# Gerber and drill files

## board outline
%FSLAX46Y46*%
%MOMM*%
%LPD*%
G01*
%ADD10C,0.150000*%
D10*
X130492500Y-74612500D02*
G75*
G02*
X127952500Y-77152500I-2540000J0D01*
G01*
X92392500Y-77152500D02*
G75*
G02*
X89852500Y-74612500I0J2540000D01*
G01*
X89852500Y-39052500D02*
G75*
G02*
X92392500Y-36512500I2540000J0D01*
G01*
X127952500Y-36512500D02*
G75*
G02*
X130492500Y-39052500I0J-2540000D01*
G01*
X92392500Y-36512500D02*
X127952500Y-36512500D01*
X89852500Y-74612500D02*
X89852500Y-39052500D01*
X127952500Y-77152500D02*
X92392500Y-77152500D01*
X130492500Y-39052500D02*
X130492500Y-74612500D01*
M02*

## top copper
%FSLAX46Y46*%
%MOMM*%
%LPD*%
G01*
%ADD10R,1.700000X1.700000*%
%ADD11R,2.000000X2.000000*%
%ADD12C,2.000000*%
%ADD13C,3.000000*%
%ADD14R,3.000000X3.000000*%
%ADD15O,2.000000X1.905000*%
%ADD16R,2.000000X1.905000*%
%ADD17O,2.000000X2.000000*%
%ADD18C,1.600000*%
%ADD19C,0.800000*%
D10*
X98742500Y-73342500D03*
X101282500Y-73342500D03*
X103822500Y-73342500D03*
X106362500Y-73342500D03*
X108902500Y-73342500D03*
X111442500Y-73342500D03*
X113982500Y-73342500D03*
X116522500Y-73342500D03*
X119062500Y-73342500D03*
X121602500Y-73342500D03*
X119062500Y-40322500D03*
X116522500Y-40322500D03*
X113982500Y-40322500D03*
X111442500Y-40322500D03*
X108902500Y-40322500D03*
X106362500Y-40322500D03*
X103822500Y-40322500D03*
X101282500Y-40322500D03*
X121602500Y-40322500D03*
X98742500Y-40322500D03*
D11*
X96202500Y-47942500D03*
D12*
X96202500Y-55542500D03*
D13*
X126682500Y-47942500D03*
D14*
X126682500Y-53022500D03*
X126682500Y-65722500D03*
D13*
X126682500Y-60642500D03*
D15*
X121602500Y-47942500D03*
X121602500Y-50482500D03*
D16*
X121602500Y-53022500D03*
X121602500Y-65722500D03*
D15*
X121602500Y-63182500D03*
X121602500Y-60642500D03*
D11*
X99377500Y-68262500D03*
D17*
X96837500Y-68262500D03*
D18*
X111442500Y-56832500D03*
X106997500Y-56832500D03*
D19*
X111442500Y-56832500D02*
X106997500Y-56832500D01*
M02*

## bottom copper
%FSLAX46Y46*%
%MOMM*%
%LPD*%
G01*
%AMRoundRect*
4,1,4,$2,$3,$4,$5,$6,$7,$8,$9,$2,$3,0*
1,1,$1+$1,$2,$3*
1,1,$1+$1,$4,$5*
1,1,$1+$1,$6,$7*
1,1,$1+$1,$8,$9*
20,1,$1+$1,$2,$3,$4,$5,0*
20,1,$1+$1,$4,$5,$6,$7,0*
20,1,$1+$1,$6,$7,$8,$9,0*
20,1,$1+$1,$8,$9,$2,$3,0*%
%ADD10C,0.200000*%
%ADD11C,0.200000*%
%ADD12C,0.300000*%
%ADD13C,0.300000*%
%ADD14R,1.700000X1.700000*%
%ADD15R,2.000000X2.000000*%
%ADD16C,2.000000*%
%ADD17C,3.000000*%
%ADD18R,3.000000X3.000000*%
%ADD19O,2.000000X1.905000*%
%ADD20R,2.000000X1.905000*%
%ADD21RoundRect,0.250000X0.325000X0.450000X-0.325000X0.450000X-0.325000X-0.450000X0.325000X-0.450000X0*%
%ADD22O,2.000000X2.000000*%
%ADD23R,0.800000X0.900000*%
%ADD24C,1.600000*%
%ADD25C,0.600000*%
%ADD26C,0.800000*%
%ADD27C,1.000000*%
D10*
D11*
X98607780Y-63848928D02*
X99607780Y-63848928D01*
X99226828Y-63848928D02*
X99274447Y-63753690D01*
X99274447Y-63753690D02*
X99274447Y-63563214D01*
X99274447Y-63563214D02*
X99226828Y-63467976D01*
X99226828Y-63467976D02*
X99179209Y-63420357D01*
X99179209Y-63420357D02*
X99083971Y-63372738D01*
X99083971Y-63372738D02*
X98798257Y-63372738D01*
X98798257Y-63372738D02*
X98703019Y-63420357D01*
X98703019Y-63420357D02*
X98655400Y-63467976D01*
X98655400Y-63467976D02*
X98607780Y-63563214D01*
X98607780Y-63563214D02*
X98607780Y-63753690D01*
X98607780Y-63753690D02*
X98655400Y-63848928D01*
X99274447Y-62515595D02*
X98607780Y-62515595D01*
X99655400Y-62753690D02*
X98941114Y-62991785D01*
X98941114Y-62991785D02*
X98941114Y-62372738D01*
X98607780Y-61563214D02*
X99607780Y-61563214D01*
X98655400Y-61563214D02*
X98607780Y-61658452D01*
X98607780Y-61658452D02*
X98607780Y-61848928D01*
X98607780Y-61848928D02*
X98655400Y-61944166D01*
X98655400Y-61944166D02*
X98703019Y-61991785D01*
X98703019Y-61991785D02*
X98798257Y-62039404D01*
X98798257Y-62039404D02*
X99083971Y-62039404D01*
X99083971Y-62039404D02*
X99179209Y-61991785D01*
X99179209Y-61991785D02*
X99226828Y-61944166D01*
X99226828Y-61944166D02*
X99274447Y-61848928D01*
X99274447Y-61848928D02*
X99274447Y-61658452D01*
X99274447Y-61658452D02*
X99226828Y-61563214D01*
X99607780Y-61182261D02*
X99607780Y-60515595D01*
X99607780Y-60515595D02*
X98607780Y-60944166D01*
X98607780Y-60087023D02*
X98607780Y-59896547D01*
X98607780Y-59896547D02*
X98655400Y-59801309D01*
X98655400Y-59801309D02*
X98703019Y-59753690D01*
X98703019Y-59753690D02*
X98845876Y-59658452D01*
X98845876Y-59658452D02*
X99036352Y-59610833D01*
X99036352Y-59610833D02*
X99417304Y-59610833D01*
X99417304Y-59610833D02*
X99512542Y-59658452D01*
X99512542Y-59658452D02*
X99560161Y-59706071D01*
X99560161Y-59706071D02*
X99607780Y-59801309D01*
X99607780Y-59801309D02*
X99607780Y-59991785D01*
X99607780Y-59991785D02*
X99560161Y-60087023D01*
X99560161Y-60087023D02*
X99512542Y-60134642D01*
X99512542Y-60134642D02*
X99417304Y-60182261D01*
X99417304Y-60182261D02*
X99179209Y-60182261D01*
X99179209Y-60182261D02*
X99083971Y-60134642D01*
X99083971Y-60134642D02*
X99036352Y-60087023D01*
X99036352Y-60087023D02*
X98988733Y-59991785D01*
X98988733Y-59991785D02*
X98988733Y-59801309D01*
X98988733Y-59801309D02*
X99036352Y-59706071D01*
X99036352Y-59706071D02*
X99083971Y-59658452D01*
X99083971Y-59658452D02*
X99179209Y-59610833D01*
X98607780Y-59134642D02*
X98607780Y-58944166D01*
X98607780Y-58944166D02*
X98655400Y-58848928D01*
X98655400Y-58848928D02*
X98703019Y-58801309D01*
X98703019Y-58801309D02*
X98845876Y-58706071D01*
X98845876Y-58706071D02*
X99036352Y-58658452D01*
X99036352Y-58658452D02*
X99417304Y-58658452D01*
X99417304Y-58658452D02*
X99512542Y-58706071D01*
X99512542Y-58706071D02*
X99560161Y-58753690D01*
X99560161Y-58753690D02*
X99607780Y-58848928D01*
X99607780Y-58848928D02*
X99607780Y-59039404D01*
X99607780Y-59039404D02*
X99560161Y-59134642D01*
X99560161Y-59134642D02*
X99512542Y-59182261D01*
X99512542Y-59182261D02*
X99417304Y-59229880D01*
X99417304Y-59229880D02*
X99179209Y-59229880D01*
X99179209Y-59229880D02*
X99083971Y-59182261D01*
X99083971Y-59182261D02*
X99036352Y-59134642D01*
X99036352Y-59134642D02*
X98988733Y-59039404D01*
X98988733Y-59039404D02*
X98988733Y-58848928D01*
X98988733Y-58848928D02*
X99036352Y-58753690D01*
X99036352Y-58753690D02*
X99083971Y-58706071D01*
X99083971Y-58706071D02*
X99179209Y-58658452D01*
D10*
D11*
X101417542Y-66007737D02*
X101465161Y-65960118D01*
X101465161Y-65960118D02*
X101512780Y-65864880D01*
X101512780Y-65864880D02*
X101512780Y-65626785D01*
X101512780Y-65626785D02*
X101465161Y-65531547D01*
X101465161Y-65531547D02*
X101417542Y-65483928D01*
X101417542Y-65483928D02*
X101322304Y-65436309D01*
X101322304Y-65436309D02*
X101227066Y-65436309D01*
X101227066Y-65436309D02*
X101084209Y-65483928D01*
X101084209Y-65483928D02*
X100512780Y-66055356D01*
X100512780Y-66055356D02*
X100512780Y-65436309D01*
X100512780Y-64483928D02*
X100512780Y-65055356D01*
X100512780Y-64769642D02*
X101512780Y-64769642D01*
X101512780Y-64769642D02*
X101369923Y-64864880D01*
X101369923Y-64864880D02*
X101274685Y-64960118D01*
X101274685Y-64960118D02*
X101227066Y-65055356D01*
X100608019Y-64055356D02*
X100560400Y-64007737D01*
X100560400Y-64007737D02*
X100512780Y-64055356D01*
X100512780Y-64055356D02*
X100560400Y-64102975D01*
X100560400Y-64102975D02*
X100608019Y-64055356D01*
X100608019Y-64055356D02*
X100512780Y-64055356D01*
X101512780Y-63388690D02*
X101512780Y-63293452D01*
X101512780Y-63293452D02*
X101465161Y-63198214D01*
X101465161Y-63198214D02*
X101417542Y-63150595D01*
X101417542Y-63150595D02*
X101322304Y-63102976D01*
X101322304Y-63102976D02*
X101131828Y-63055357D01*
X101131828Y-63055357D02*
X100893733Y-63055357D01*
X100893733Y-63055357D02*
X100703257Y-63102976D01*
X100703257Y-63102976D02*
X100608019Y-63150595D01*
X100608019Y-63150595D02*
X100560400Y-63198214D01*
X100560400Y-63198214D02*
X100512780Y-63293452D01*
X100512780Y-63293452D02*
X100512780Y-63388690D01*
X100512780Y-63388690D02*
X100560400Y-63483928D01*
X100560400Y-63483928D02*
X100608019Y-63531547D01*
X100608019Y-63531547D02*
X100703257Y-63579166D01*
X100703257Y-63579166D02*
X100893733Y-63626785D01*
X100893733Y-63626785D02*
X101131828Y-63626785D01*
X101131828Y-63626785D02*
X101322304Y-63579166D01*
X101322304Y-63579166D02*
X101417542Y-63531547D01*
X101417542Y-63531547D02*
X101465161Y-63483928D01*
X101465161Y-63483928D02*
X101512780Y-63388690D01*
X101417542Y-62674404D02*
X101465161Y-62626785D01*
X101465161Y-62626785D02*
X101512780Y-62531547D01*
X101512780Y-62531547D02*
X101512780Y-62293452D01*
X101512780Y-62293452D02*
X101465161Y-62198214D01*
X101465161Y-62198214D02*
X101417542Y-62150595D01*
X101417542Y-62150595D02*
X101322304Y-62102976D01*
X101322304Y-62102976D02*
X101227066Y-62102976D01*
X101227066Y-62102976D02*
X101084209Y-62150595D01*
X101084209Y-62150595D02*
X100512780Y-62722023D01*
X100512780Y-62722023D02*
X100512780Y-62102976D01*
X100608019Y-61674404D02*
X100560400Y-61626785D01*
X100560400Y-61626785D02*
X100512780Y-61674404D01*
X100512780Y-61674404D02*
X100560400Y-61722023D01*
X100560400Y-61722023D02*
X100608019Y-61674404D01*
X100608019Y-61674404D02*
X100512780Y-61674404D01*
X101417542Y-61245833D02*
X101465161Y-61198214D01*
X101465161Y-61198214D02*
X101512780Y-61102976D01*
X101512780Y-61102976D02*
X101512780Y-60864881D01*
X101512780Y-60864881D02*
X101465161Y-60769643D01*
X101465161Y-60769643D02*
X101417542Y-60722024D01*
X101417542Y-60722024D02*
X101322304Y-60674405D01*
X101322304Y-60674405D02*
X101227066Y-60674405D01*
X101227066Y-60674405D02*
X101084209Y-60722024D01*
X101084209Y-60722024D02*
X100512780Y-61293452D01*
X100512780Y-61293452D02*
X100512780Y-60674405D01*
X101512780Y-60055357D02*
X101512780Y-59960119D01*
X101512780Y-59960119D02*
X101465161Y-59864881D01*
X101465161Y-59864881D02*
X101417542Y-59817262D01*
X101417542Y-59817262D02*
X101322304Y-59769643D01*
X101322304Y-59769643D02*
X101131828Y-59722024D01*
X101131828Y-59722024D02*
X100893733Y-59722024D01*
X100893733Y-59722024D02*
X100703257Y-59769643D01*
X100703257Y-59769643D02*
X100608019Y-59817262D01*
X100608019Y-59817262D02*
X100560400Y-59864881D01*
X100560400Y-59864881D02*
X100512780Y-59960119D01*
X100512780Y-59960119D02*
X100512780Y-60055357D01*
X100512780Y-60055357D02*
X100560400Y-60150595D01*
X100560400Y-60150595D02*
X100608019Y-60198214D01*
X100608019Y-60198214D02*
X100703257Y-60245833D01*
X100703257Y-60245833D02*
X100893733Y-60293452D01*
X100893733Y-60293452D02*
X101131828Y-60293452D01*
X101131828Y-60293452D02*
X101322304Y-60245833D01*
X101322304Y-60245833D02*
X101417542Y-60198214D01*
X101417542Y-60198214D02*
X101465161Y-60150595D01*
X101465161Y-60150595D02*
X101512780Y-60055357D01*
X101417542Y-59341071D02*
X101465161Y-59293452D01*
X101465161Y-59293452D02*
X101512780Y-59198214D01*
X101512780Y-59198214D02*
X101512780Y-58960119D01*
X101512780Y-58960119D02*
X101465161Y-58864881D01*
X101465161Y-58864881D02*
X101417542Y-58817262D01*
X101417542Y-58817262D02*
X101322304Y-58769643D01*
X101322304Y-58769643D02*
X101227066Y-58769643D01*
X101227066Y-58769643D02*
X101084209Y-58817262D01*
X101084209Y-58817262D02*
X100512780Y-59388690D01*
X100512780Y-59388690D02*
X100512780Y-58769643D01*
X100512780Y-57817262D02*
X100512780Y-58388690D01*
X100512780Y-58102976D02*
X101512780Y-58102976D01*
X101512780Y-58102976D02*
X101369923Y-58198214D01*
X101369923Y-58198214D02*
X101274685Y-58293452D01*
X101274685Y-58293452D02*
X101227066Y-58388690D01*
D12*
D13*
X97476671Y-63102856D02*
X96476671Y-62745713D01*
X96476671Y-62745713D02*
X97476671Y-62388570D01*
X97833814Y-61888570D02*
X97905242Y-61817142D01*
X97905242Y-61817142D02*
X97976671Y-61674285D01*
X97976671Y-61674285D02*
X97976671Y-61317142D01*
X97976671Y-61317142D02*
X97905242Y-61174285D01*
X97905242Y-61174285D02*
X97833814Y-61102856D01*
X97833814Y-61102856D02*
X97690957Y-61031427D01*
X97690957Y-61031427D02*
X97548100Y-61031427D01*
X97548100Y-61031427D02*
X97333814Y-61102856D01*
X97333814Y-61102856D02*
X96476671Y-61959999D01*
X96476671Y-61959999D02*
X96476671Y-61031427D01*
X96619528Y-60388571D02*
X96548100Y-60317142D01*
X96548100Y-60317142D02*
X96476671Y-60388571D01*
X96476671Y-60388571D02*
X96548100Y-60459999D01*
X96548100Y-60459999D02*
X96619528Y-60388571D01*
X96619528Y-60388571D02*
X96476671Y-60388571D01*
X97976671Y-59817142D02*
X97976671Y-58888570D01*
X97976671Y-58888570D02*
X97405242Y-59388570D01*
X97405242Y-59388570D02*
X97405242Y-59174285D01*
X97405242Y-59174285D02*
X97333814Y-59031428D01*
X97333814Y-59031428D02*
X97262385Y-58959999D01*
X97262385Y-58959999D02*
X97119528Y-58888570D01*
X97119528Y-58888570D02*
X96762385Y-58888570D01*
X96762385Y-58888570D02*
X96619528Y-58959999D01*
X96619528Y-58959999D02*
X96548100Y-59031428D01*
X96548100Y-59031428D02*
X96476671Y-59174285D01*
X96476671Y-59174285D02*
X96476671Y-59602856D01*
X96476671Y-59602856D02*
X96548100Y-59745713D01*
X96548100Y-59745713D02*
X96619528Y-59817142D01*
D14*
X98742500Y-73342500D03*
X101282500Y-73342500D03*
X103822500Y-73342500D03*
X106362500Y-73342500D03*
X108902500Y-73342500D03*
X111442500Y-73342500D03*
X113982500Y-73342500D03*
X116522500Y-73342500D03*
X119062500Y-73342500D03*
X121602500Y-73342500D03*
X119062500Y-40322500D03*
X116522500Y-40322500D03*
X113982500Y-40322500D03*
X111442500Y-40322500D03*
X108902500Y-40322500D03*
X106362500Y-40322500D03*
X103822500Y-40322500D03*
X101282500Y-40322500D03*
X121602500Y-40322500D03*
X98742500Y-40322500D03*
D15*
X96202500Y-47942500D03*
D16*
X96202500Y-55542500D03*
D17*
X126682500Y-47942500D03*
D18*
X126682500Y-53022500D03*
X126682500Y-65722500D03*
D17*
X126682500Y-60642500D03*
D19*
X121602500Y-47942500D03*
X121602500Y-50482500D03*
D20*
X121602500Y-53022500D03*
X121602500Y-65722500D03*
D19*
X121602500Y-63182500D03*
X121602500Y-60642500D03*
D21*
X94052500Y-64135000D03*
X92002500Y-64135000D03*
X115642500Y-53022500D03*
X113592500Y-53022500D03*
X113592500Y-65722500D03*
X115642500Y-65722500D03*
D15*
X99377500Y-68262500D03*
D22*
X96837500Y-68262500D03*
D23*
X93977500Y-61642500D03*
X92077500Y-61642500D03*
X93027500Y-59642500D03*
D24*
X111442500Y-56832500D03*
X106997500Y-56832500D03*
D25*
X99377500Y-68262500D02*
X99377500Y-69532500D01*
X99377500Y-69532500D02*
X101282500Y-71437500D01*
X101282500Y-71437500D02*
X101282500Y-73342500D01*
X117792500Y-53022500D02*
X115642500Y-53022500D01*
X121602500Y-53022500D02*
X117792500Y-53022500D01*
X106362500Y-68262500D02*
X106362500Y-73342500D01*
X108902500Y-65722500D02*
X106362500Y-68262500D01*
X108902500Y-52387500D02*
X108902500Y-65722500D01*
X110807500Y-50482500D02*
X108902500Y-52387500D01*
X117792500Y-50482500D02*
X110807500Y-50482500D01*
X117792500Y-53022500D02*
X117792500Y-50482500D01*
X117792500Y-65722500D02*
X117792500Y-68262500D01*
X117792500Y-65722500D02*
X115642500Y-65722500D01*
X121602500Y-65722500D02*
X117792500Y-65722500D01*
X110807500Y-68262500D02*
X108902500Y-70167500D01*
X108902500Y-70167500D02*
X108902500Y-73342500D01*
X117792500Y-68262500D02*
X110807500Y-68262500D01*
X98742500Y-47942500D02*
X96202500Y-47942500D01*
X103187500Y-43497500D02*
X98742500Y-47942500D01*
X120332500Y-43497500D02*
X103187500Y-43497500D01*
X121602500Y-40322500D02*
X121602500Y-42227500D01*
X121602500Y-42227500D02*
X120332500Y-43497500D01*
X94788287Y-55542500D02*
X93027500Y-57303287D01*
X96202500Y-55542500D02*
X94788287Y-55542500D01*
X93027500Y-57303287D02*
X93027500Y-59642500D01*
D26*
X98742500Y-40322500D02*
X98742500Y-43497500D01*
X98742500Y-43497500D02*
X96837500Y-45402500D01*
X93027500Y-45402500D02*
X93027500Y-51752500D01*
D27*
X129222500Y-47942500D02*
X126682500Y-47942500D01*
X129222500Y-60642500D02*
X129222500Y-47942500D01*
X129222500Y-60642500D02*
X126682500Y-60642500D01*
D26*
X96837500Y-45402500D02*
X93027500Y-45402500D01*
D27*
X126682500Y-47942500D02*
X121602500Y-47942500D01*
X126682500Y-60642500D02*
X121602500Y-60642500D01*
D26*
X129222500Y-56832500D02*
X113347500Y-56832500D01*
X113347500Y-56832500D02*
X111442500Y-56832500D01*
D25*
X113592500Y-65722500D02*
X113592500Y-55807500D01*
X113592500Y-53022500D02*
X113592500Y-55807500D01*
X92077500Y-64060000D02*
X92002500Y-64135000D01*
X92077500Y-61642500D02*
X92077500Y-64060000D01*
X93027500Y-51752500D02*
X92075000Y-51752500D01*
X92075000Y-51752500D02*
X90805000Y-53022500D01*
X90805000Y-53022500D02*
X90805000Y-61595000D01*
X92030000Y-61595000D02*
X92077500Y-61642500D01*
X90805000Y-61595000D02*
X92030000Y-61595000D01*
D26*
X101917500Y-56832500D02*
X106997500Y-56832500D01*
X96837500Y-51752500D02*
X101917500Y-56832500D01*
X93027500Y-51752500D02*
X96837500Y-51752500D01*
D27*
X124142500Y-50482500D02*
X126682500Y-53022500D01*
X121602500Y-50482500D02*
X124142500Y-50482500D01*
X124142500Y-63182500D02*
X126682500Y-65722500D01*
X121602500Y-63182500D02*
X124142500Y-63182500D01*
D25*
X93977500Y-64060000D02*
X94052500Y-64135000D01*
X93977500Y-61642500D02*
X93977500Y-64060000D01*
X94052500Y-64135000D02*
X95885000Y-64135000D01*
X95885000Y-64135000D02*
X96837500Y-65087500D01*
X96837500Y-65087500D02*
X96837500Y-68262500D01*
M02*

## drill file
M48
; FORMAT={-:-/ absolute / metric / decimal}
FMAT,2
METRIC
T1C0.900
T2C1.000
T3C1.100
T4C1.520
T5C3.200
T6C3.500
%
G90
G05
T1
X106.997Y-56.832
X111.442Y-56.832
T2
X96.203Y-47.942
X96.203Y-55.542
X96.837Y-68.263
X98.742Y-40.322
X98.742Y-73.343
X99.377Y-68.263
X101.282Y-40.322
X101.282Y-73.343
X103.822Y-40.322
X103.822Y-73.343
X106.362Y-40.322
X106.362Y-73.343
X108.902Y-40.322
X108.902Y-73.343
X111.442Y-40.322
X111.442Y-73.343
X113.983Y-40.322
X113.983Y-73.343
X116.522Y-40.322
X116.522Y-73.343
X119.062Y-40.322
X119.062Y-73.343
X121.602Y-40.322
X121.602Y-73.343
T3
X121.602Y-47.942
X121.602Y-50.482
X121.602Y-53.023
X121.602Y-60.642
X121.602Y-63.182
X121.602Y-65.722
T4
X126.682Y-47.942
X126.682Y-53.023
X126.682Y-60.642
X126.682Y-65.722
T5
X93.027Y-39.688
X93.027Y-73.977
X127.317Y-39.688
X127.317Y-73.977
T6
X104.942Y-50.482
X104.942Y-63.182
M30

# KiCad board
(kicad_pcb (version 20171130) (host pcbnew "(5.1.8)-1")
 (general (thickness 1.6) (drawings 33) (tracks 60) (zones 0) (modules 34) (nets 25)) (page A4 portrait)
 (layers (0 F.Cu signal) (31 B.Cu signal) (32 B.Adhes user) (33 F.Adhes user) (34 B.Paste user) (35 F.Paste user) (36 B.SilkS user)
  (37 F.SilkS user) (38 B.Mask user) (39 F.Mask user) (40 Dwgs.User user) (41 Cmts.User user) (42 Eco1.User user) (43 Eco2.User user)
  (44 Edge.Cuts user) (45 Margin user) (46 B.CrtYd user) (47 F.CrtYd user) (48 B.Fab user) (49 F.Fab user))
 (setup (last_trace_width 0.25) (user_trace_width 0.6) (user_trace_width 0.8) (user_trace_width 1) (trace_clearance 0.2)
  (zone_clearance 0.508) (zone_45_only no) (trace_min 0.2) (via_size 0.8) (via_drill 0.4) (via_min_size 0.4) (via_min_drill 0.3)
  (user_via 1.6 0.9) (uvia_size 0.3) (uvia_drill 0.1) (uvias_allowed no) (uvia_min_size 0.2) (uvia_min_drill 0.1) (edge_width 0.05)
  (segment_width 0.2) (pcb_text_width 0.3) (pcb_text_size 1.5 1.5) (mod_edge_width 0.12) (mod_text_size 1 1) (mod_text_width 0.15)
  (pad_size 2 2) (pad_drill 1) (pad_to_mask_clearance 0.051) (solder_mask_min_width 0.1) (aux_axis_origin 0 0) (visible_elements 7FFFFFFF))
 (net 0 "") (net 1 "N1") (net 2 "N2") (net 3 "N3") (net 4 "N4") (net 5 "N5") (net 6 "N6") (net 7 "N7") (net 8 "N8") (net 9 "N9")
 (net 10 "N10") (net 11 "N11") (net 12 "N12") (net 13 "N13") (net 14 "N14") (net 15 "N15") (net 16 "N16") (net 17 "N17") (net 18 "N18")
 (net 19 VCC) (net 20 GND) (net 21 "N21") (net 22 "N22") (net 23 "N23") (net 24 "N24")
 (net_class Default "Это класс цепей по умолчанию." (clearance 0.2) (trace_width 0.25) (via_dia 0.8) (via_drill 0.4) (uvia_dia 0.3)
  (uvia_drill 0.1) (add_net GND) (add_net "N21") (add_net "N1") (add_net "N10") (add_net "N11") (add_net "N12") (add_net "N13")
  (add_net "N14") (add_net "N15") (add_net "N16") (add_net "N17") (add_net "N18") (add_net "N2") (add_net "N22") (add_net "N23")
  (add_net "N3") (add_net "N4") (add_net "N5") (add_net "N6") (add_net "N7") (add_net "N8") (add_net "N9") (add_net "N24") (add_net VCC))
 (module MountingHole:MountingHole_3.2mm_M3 (layer F.Cu) (at 127.3175 39.6875 270)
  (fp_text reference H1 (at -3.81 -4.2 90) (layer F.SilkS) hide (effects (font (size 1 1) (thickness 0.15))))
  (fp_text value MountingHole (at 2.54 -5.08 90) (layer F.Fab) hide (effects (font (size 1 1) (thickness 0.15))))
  (pad 1 np_thru_hole circle (at 0 0 270) (size 3.2 3.2) (drill 3.2) (layers *.Cu *.Mask)))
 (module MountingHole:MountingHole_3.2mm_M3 (layer F.Cu) (at 93.0275 39.6875 270)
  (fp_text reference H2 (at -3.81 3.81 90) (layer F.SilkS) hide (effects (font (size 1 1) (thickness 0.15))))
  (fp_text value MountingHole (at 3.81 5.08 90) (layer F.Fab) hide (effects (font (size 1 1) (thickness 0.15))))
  (pad 1 np_thru_hole circle (at 0 0 270) (size 3.2 3.2) (drill 3.2) (layers *.Cu *.Mask)))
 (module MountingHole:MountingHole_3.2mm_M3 (layer F.Cu) (at 127.3175 73.9775 270)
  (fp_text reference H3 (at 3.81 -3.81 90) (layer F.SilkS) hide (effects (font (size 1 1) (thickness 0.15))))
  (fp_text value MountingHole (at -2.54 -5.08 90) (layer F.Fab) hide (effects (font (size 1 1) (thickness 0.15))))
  (pad 1 np_thru_hole circle (at 0 0 270) (size 3.2 3.2) (drill 3.2) (layers *.Cu *.Mask)))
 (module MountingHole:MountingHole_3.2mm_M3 (layer F.Cu) (at 93.0275 73.9775 270)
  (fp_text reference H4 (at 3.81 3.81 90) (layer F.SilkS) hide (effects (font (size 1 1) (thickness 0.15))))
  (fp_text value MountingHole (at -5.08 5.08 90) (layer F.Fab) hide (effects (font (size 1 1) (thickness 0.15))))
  (pad 1 np_thru_hole circle (at 0 0 270) (size 3.2 3.2) (drill 3.2) (layers *.Cu *.Mask)))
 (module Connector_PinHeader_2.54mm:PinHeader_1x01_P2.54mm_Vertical (layer F.Cu) (at 98.7425 73.3425 270)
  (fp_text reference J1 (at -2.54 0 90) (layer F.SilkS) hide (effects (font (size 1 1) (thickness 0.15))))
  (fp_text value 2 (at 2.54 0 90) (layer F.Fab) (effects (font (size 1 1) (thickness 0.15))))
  (pad 1 thru_hole rect (at 0 0 270) (size 1.7 1.7) (drill 1) (layers *.Cu *.Mask) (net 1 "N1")))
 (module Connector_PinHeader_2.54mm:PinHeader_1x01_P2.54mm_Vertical (layer F.Cu) (at 101.2825 73.3425 270)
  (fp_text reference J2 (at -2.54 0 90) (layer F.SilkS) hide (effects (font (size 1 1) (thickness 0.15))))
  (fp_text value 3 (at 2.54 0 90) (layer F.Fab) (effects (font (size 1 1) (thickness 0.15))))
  (pad 1 thru_hole rect (at 0 0 270) (size 1.7 1.7) (drill 1) (layers *.Cu *.Mask) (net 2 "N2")))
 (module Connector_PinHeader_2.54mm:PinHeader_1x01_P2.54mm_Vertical (layer F.Cu) (at 103.8225 73.3425 270)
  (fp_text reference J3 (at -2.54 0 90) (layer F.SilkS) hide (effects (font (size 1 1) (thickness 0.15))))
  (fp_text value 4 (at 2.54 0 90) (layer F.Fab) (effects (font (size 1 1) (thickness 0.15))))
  (pad 1 thru_hole rect (at 0 0 270) (size 1.7 1.7) (drill 1) (layers *.Cu *.Mask) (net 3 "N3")))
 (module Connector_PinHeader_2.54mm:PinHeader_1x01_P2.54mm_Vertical (layer F.Cu) (at 106.3625 73.3425 270)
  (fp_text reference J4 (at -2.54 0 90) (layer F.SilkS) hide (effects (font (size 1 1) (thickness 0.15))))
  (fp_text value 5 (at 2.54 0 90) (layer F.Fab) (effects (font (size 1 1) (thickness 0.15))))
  (pad 1 thru_hole rect (at 0 0 270) (size 1.7 1.7) (drill 1) (layers *.Cu *.Mask) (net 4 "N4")))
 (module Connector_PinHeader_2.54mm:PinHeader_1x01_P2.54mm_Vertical (layer F.Cu) (at 108.9025 73.3425 270)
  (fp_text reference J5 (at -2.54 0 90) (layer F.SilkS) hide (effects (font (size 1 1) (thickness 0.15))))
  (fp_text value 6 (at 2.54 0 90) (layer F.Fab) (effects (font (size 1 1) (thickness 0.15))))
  (pad 1 thru_hole rect (at 0 0 270) (size 1.7 1.7) (drill 1) (layers *.Cu *.Mask) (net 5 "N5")))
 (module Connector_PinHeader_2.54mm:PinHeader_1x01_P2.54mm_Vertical (layer F.Cu) (at 111.4425 73.3425 270)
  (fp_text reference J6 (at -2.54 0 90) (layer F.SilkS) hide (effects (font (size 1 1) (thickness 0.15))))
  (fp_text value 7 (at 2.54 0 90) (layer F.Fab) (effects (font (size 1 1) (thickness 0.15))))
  (pad 1 thru_hole rect (at 0 0 270) (size 1.7 1.7) (drill 1) (layers *.Cu *.Mask) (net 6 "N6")))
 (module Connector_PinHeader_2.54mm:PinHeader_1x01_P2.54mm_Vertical (layer F.Cu) (at 113.9825 73.3425 270)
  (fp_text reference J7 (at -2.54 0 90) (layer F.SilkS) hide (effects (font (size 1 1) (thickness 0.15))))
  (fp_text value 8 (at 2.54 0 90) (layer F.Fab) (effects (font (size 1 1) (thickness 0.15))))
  (pad 1 thru_hole rect (at 0 0 270) (size 1.7 1.7) (drill 1) (layers *.Cu *.Mask) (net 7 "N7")))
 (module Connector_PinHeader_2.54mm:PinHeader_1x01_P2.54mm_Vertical (layer F.Cu) (at 116.5225 73.3425 270)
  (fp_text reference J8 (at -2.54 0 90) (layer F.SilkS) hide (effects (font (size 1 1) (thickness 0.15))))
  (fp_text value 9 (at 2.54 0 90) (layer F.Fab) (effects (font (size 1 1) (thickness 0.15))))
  (pad 1 thru_hole rect (at 0 0 270) (size 1.7 1.7) (drill 1) (layers *.Cu *.Mask) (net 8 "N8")))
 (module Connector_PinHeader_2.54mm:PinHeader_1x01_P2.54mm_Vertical (layer F.Cu) (at 119.0625 73.3425 270)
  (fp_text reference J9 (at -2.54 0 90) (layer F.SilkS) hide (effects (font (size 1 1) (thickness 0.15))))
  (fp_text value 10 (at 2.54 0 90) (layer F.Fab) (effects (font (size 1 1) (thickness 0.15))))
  (pad 1 thru_hole rect (at 0 0 270) (size 1.7 1.7) (drill 1) (layers *.Cu *.Mask) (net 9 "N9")))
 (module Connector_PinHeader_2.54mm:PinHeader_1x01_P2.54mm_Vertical (layer F.Cu) (at 121.6025 73.3425 270)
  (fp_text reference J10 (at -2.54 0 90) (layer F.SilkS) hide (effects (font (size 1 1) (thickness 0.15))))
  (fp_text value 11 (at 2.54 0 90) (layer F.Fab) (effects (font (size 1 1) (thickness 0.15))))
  (pad 1 thru_hole rect (at 0 0 270) (size 1.7 1.7) (drill 1) (layers *.Cu *.Mask) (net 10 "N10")))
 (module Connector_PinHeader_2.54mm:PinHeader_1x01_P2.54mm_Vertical (layer F.Cu) (at 119.0625 40.3225 270)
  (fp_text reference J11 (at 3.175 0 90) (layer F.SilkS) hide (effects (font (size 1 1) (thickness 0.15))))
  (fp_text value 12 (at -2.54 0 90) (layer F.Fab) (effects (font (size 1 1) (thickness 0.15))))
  (pad 1 thru_hole rect (at 0 0 270) (size 1.7 1.7) (drill 1) (layers *.Cu *.Mask) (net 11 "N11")))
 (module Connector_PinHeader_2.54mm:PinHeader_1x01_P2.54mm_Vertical (layer F.Cu) (at 116.5225 40.3225 270)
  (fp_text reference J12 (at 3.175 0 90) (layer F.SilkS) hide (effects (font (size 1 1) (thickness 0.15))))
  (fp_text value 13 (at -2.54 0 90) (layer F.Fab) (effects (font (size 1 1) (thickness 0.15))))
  (pad 1 thru_hole rect (at 0 0 270) (size 1.7 1.7) (drill 1) (layers *.Cu *.Mask) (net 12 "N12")))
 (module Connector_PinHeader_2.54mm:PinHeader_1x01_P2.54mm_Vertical (layer F.Cu) (at 113.9825 40.3225 270)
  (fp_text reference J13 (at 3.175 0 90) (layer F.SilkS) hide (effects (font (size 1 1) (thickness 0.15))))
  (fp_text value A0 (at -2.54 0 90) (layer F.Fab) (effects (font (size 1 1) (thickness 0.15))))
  (pad 1 thru_hole rect (at 0 0 270) (size 1.7 1.7) (drill 1) (layers *.Cu *.Mask) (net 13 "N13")))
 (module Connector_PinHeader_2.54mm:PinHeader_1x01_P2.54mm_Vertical (layer F.Cu) (at 111.4425 40.3225 270)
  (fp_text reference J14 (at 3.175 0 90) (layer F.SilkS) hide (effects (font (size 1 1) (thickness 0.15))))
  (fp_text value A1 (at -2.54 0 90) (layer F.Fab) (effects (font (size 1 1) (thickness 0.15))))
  (pad 1 thru_hole rect (at 0 0 270) (size 1.7 1.7) (drill 1) (layers *.Cu *.Mask) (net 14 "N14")))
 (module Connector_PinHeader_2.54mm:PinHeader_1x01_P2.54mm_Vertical (layer F.Cu) (at 108.9025 40.3225 270)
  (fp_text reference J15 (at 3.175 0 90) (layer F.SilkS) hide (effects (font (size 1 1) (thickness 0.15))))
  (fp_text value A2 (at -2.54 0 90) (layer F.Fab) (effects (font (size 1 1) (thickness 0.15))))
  (pad 1 thru_hole rect (at 0 0 270) (size 1.7 1.7) (drill 1) (layers *.Cu *.Mask) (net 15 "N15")))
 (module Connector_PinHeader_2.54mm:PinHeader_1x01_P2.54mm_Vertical (layer F.Cu) (at 106.3625 40.3225 270)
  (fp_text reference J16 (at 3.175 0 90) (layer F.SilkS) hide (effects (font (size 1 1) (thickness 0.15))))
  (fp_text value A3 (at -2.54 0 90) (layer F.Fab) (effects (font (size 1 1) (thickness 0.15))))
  (pad 1 thru_hole rect (at 0 0 270) (size 1.7 1.7) (drill 1) (layers *.Cu *.Mask) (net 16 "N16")))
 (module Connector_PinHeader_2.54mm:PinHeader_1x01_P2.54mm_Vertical (layer F.Cu) (at 103.8225 40.3225 270)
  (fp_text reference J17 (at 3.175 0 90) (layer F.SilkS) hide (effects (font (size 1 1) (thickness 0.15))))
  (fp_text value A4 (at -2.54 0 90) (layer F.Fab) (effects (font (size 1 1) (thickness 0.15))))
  (pad 1 thru_hole rect (at 0 0 270) (size 1.7 1.7) (drill 1) (layers *.Cu *.Mask) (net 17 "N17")))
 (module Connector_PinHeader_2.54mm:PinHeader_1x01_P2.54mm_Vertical (layer F.Cu) (at 101.2825 40.3225 270)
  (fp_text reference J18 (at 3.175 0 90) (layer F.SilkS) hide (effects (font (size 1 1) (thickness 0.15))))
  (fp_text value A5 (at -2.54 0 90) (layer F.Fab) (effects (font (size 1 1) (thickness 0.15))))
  (pad 1 thru_hole rect (at 0 0 270) (size 1.7 1.7) (drill 1) (layers *.Cu *.Mask) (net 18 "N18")))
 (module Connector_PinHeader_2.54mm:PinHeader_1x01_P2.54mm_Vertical (layer F.Cu) (at 121.6025 40.3225 270)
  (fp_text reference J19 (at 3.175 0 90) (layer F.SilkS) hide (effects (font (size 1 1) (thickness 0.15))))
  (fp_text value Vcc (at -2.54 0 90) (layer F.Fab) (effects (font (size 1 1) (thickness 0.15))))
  (pad 1 thru_hole rect (at 0 0 270) (size 1.7 1.7) (drill 1) (layers *.Cu *.Mask) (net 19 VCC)))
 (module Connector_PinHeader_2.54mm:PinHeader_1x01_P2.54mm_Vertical (layer F.Cu) (at 98.7425 40.3225 270)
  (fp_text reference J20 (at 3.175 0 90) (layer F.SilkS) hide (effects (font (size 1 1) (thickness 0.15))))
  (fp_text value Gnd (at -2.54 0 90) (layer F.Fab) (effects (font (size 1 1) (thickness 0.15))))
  (pad 1 thru_hole rect (at 0 0 270) (size 1.7 1.7) (drill 1) (layers *.Cu *.Mask) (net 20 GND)))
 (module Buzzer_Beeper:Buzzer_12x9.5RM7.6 (layer F.Cu) (at 96.2025 47.9425 270)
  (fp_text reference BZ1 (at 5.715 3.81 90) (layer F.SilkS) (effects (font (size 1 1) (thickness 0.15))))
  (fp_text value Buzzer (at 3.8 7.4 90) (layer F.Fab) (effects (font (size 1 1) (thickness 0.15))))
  (pad 1 thru_hole rect (at 0 0 270) (size 2 2) (drill 1) (layers *.Cu *.Mask) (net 19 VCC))
  (pad 2 thru_hole circle (at 7.6 0 270) (size 2 2) (drill 1) (layers *.Cu *.Mask) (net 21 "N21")))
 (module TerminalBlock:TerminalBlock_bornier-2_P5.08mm (layer F.Cu) (at 126.6825 53.0225 90)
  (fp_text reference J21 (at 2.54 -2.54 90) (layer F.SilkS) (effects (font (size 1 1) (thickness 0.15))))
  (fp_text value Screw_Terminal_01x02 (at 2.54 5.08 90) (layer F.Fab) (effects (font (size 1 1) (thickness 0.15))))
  (pad 2 thru_hole circle (at 5.08 0 90) (size 3 3) (drill 1.52) (layers *.Cu *.Mask) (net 20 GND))
  (pad 1 thru_hole rect (at 0 0 90) (size 3 3) (drill 1.52) (layers *.Cu *.Mask) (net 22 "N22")))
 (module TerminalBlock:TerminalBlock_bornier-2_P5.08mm (layer F.Cu) (at 126.6825 65.7225 90)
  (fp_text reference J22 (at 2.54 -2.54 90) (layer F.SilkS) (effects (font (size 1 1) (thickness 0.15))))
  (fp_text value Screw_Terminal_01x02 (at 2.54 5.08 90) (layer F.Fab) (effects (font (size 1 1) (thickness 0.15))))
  (pad 1 thru_hole rect (at 0 0 90) (size 3 3) (drill 1.52) (layers *.Cu *.Mask) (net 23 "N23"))
  (pad 2 thru_hole circle (at 5.08 0 90) (size 3 3) (drill 1.52) (layers *.Cu *.Mask) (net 20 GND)))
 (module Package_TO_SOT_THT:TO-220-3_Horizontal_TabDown (layer F.Cu) (at 121.6025 53.0225 90)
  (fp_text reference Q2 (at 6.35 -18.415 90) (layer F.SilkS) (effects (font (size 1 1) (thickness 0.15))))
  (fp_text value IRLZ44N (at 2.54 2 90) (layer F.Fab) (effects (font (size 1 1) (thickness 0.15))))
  (pad 3 thru_hole oval (at 5.08 0 90) (size 1.905 2) (drill 1.1) (layers *.Cu *.Mask) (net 20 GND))
  (pad 2 thru_hole oval (at 2.54 0 90) (size 1.905 2) (drill 1.1) (layers *.Cu *.Mask) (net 22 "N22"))
  (pad 1 thru_hole rect (at 0 0 90) (size 1.905 2) (drill 1.1) (layers *.Cu *.Mask) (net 4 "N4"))
  (pad "" np_thru_hole oval (at 2.54 -16.66 90) (size 3.5 3.5) (drill 3.5) (layers *.Cu *.Mask)))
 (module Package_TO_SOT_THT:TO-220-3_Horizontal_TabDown (layer F.Cu) (at 121.6025 65.7225 90)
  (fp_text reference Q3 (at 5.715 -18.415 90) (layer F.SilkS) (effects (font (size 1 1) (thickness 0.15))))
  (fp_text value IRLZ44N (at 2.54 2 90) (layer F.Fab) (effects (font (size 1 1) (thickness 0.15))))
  (pad "" np_thru_hole oval (at 2.54 -16.66 90) (size 3.5 3.5) (drill 3.5) (layers *.Cu *.Mask))
  (pad 1 thru_hole rect (at 0 0 90) (size 1.905 2) (drill 1.1) (layers *.Cu *.Mask) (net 5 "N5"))
  (pad 2 thru_hole oval (at 2.54 0 90) (size 1.905 2) (drill 1.1) (layers *.Cu *.Mask) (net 23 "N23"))
  (pad 3 thru_hole oval (at 5.08 0 90) (size 1.905 2) (drill 1.1) (layers *.Cu *.Mask) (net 20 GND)))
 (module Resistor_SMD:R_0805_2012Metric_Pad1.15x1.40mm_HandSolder (layer B.Cu) (at 93.0275 64.135 180)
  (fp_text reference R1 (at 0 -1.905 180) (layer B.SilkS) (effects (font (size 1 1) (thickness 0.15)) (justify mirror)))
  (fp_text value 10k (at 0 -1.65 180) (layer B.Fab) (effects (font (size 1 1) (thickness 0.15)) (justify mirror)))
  (pad 1 smd roundrect (at -1.025 0 180) (size 1.15 1.4) (layers B.Cu B.Paste B.Mask) (roundrect_rratio 0.217391) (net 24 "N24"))
  (pad 2 smd roundrect (at 1.025 0 180) (size 1.15 1.4) (layers B.Cu B.Paste B.Mask) (roundrect_rratio 0.217391) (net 20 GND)))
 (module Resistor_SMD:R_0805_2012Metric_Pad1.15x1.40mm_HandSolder (layer B.Cu) (at 114.6175 53.0225 180)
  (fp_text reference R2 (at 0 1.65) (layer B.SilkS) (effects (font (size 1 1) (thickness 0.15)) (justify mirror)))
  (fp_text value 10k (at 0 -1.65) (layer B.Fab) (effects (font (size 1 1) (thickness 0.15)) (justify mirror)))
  (pad 1 smd roundrect (at -1.025 0 180) (size 1.15 1.4) (layers B.Cu B.Paste B.Mask) (roundrect_rratio 0.217391) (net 4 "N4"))
  (pad 2 smd roundrect (at 1.025 0 180) (size 1.15 1.4) (layers B.Cu B.Paste B.Mask) (roundrect_rratio 0.217391) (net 20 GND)))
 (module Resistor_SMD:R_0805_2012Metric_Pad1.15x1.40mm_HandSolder (layer B.Cu) (at 114.6175 65.7225 180)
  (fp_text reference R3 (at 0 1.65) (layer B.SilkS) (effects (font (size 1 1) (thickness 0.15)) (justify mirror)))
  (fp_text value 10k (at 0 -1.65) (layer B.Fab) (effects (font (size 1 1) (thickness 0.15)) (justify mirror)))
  (pad 2 smd roundrect (at 1.025 0 180) (size 1.15 1.4) (layers B.Cu B.Paste B.Mask) (roundrect_rratio 0.217391) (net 20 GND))
  (pad 1 smd roundrect (at -1.025 0 180) (size 1.15 1.4) (layers B.Cu B.Paste B.Mask) (roundrect_rratio 0.217391) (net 5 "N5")))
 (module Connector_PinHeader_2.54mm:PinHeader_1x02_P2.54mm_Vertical (layer F.Cu) (at 99.3775 68.2625 270)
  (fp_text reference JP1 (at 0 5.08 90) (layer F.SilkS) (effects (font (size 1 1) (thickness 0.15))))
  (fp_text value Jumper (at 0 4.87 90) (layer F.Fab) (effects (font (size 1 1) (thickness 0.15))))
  (pad 1 thru_hole rect (at 0 0 270) (size 2 2) (drill 1) (layers *.Cu *.Mask) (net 2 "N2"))
  (pad 2 thru_hole oval (at 0 2.54 270) (size 2 2) (drill 1) (layers *.Cu *.Mask) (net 24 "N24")))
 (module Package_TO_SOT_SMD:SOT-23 (layer B.Cu) (at 93.0275 60.6425 90)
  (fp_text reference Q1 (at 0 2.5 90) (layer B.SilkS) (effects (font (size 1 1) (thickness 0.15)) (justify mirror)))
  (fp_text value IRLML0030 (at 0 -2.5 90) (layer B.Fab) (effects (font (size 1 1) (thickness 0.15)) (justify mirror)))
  (pad 1 smd rect (at -1 0.95 90) (size 0.9 0.8) (layers B.Cu B.Paste B.Mask) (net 24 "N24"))
  (pad 2 smd rect (at -1 -0.95 90) (size 0.9 0.8) (layers B.Cu B.Paste B.Mask) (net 20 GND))
  (pad 3 smd rect (at 1 0 90) (size 0.9 0.8) (layers B.Cu B.Paste B.Mask) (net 21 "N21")))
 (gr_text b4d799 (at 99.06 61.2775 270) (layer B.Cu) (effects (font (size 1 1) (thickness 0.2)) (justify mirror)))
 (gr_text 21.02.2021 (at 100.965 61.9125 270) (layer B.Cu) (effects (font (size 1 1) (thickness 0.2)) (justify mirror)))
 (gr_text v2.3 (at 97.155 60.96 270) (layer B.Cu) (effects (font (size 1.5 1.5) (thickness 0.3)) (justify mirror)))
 (gr_arc (start 127.9525 74.6125) (end 127.9525 77.1525) (angle -90) (layer Edge.Cuts) (width 0.15))
 (gr_arc (start 92.3925 74.6125) (end 89.8525 74.6125) (angle -90) (layer Edge.Cuts) (width 0.15))
 (gr_arc (start 92.3925 39.0525) (end 92.3925 36.5125) (angle -90) (layer Edge.Cuts) (width 0.15))
 (gr_arc (start 127.9525 39.0525) (end 130.4925 39.0525) (angle -90) (layer Edge.Cuts) (width 0.15))
 (gr_line (start 92.3925 36.5125) (end 127.9525 36.5125) (layer Edge.Cuts) (width 0.15))
 (gr_line (start 89.8525 74.6125) (end 89.8525 39.0525) (layer Edge.Cuts) (width 0.15))
 (gr_line (start 127.9525 77.1525) (end 92.3925 77.1525) (layer Edge.Cuts) (width 0.15))
 (gr_line (start 130.4925 39.0525) (end 130.4925 74.6125) (layer Edge.Cuts) (width 0.15))
 (segment (start 99.3775 68.2625) (end 99.3775 69.5325) (width 0.6) (layer B.Cu) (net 2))
 (segment (start 99.3775 69.5325) (end 101.2825 71.4375) (width 0.6) (layer B.Cu) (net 2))
 (segment (start 101.2825 71.4375) (end 101.2825 73.3425) (width 0.6) (layer B.Cu) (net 2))
 (segment (start 117.7925 53.0225) (end 115.6425 53.0225) (width 0.6) (layer B.Cu) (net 4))
 (segment (start 121.6025 53.0225) (end 117.7925 53.0225) (width 0.6) (layer B.Cu) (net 4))
 (segment (start 106.3625 68.2625) (end 106.3625 73.3425) (width 0.6) (layer B.Cu) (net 4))
 (segment (start 108.9025 65.7225) (end 106.3625 68.2625) (width 0.6) (layer B.Cu) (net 4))
 (segment (start 108.9025 52.3875) (end 108.9025 65.7225) (width 0.6) (layer B.Cu) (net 4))
 (segment (start 110.8075 50.4825) (end 108.9025 52.3875) (width 0.6) (layer B.Cu) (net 4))
 (segment (start 117.7925 50.4825) (end 110.8075 50.4825) (width 0.6) (layer B.Cu) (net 4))
 (segment (start 117.7925 53.0225) (end 117.7925 50.4825) (width 0.6) (layer B.Cu) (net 4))
 (segment (start 117.7925 65.7225) (end 117.7925 68.2625) (width 0.6) (layer B.Cu) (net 5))
 (segment (start 117.7925 65.7225) (end 115.6425 65.7225) (width 0.6) (layer B.Cu) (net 5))
 (segment (start 121.6025 65.7225) (end 117.7925 65.7225) (width 0.6) (layer B.Cu) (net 5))
 (segment (start 110.8075 68.2625) (end 108.9025 70.1675) (width 0.6) (layer B.Cu) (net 5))
 (segment (start 108.9025 70.1675) (end 108.9025 73.3425) (width 0.6) (layer B.Cu) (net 5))
 (segment (start 117.7925 68.2625) (end 110.8075 68.2625) (width 0.6) (layer B.Cu) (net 5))
 (segment (start 98.7425 47.9425) (end 96.2025 47.9425) (width 0.6) (layer B.Cu) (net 19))
 (segment (start 103.1875 43.4975) (end 98.7425 47.9425) (width 0.6) (layer B.Cu) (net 19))
 (segment (start 120.3325 43.4975) (end 103.1875 43.4975) (width 0.6) (layer B.Cu) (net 19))
 (segment (start 121.6025 40.3225) (end 121.6025 42.2275) (width 0.6) (layer B.Cu) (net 19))
 (segment (start 121.6025 42.2275) (end 120.3325 43.4975) (width 0.6) (layer B.Cu) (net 19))
 (segment (start 94.788287 55.5425) (end 93.0275 57.303287) (width 0.6) (layer B.Cu) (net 21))
 (segment (start 96.2025 55.5425) (end 94.788287 55.5425) (width 0.6) (layer B.Cu) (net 21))
 (segment (start 93.0275 57.303287) (end 93.0275 59.6425) (width 0.6) (layer B.Cu) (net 21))
 (segment (start 98.7425 40.3225) (end 98.7425 43.4975) (width 0.8) (layer B.Cu) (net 20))
 (segment (start 98.7425 43.4975) (end 96.8375 45.4025) (width 0.8) (layer B.Cu) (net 20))
 (segment (start 93.0275 45.4025) (end 93.0275 51.7525) (width 0.8) (layer B.Cu) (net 20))
 (via (at 111.4425 56.8325) (size 1.6) (drill 0.9) (layers F.Cu B.Cu) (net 20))
 (via (at 106.9975 56.8325) (size 1.6) (drill 0.9) (layers F.Cu B.Cu) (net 20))
 (segment (start 111.4425 56.8325) (end 106.9975 56.8325) (width 0.8) (layer F.Cu) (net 20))
 (segment (start 129.2225 47.9425) (end 126.6825 47.9425) (width 1) (layer B.Cu) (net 20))
 (segment (start 129.2225 60.6425) (end 129.2225 47.9425) (width 1) (layer B.Cu) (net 20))
 (segment (start 129.2225 60.6425) (end 126.6825 60.6425) (width 1) (layer B.Cu) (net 20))
 (segment (start 96.8375 45.4025) (end 93.0275 45.4025) (width 0.8) (layer B.Cu) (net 20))
 (segment (start 126.6825 47.9425) (end 121.6025 47.9425) (width 1) (layer B.Cu) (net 20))
 (segment (start 126.6825 60.6425) (end 121.6025 60.6425) (width 1) (layer B.Cu) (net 20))
 (segment (start 129.2225 56.8325) (end 113.3475 56.8325) (width 0.8) (layer B.Cu) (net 20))
 (segment (start 113.3475 56.8325) (end 111.4425 56.8325) (width 0.8) (layer B.Cu) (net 20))
 (segment (start 113.5925 65.7225) (end 113.5925 55.8075) (width 0.6) (layer B.Cu) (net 20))
 (segment (start 113.5925 53.0225) (end 113.5925 55.8075) (width 0.6) (layer B.Cu) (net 20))
 (segment (start 92.0775 64.06) (end 92.0025 64.135) (width 0.6) (layer B.Cu) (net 20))
 (segment (start 92.0775 61.6425) (end 92.0775 64.06) (width 0.6) (layer B.Cu) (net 20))
 (segment (start 93.0275 51.7525) (end 92.075 51.7525) (width 0.6) (layer B.Cu) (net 20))
 (segment (start 92.075 51.7525) (end 90.805 53.0225) (width 0.6) (layer B.Cu) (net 20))
 (segment (start 90.805 53.0225) (end 90.805 61.595) (width 0.6) (layer B.Cu) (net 20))
 (segment (start 92.03 61.595) (end 92.0775 61.6425) (width 0.6) (layer B.Cu) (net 20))
 (segment (start 90.805 61.595) (end 92.03 61.595) (width 0.6) (layer B.Cu) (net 20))
 (segment (start 101.9175 56.8325) (end 106.9975 56.8325) (width 0.8) (layer B.Cu) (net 20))
 (segment (start 96.8375 51.7525) (end 101.9175 56.8325) (width 0.8) (layer B.Cu) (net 20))
 (segment (start 93.0275 51.7525) (end 96.8375 51.7525) (width 0.8) (layer B.Cu) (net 20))
 (segment (start 124.1425 50.4825) (end 126.6825 53.0225) (width 1) (layer B.Cu) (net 22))
 (segment (start 121.6025 50.4825) (end 124.1425 50.4825) (width 1) (layer B.Cu) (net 22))
 (segment (start 124.1425 63.1825) (end 126.6825 65.7225) (width 1) (layer B.Cu) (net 23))
 (segment (start 121.6025 63.1825) (end 124.1425 63.1825) (width 1) (layer B.Cu) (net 23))
 (segment (start 93.9775 64.06) (end 94.0525 64.135) (width 0.6) (layer B.Cu) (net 24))
 (segment (start 93.9775 61.6425) (end 93.9775 64.06) (width 0.6) (layer B.Cu) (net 24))
 (segment (start 94.0525 64.135) (end 95.885 64.135) (width 0.6) (layer B.Cu) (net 24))
 (segment (start 95.885 64.135) (end 96.8375 65.0875) (width 0.6) (layer B.Cu) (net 24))
 (segment (start 96.8375 65.0875) (end 96.8375 68.2625) (width 0.6) (layer B.Cu) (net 24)))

